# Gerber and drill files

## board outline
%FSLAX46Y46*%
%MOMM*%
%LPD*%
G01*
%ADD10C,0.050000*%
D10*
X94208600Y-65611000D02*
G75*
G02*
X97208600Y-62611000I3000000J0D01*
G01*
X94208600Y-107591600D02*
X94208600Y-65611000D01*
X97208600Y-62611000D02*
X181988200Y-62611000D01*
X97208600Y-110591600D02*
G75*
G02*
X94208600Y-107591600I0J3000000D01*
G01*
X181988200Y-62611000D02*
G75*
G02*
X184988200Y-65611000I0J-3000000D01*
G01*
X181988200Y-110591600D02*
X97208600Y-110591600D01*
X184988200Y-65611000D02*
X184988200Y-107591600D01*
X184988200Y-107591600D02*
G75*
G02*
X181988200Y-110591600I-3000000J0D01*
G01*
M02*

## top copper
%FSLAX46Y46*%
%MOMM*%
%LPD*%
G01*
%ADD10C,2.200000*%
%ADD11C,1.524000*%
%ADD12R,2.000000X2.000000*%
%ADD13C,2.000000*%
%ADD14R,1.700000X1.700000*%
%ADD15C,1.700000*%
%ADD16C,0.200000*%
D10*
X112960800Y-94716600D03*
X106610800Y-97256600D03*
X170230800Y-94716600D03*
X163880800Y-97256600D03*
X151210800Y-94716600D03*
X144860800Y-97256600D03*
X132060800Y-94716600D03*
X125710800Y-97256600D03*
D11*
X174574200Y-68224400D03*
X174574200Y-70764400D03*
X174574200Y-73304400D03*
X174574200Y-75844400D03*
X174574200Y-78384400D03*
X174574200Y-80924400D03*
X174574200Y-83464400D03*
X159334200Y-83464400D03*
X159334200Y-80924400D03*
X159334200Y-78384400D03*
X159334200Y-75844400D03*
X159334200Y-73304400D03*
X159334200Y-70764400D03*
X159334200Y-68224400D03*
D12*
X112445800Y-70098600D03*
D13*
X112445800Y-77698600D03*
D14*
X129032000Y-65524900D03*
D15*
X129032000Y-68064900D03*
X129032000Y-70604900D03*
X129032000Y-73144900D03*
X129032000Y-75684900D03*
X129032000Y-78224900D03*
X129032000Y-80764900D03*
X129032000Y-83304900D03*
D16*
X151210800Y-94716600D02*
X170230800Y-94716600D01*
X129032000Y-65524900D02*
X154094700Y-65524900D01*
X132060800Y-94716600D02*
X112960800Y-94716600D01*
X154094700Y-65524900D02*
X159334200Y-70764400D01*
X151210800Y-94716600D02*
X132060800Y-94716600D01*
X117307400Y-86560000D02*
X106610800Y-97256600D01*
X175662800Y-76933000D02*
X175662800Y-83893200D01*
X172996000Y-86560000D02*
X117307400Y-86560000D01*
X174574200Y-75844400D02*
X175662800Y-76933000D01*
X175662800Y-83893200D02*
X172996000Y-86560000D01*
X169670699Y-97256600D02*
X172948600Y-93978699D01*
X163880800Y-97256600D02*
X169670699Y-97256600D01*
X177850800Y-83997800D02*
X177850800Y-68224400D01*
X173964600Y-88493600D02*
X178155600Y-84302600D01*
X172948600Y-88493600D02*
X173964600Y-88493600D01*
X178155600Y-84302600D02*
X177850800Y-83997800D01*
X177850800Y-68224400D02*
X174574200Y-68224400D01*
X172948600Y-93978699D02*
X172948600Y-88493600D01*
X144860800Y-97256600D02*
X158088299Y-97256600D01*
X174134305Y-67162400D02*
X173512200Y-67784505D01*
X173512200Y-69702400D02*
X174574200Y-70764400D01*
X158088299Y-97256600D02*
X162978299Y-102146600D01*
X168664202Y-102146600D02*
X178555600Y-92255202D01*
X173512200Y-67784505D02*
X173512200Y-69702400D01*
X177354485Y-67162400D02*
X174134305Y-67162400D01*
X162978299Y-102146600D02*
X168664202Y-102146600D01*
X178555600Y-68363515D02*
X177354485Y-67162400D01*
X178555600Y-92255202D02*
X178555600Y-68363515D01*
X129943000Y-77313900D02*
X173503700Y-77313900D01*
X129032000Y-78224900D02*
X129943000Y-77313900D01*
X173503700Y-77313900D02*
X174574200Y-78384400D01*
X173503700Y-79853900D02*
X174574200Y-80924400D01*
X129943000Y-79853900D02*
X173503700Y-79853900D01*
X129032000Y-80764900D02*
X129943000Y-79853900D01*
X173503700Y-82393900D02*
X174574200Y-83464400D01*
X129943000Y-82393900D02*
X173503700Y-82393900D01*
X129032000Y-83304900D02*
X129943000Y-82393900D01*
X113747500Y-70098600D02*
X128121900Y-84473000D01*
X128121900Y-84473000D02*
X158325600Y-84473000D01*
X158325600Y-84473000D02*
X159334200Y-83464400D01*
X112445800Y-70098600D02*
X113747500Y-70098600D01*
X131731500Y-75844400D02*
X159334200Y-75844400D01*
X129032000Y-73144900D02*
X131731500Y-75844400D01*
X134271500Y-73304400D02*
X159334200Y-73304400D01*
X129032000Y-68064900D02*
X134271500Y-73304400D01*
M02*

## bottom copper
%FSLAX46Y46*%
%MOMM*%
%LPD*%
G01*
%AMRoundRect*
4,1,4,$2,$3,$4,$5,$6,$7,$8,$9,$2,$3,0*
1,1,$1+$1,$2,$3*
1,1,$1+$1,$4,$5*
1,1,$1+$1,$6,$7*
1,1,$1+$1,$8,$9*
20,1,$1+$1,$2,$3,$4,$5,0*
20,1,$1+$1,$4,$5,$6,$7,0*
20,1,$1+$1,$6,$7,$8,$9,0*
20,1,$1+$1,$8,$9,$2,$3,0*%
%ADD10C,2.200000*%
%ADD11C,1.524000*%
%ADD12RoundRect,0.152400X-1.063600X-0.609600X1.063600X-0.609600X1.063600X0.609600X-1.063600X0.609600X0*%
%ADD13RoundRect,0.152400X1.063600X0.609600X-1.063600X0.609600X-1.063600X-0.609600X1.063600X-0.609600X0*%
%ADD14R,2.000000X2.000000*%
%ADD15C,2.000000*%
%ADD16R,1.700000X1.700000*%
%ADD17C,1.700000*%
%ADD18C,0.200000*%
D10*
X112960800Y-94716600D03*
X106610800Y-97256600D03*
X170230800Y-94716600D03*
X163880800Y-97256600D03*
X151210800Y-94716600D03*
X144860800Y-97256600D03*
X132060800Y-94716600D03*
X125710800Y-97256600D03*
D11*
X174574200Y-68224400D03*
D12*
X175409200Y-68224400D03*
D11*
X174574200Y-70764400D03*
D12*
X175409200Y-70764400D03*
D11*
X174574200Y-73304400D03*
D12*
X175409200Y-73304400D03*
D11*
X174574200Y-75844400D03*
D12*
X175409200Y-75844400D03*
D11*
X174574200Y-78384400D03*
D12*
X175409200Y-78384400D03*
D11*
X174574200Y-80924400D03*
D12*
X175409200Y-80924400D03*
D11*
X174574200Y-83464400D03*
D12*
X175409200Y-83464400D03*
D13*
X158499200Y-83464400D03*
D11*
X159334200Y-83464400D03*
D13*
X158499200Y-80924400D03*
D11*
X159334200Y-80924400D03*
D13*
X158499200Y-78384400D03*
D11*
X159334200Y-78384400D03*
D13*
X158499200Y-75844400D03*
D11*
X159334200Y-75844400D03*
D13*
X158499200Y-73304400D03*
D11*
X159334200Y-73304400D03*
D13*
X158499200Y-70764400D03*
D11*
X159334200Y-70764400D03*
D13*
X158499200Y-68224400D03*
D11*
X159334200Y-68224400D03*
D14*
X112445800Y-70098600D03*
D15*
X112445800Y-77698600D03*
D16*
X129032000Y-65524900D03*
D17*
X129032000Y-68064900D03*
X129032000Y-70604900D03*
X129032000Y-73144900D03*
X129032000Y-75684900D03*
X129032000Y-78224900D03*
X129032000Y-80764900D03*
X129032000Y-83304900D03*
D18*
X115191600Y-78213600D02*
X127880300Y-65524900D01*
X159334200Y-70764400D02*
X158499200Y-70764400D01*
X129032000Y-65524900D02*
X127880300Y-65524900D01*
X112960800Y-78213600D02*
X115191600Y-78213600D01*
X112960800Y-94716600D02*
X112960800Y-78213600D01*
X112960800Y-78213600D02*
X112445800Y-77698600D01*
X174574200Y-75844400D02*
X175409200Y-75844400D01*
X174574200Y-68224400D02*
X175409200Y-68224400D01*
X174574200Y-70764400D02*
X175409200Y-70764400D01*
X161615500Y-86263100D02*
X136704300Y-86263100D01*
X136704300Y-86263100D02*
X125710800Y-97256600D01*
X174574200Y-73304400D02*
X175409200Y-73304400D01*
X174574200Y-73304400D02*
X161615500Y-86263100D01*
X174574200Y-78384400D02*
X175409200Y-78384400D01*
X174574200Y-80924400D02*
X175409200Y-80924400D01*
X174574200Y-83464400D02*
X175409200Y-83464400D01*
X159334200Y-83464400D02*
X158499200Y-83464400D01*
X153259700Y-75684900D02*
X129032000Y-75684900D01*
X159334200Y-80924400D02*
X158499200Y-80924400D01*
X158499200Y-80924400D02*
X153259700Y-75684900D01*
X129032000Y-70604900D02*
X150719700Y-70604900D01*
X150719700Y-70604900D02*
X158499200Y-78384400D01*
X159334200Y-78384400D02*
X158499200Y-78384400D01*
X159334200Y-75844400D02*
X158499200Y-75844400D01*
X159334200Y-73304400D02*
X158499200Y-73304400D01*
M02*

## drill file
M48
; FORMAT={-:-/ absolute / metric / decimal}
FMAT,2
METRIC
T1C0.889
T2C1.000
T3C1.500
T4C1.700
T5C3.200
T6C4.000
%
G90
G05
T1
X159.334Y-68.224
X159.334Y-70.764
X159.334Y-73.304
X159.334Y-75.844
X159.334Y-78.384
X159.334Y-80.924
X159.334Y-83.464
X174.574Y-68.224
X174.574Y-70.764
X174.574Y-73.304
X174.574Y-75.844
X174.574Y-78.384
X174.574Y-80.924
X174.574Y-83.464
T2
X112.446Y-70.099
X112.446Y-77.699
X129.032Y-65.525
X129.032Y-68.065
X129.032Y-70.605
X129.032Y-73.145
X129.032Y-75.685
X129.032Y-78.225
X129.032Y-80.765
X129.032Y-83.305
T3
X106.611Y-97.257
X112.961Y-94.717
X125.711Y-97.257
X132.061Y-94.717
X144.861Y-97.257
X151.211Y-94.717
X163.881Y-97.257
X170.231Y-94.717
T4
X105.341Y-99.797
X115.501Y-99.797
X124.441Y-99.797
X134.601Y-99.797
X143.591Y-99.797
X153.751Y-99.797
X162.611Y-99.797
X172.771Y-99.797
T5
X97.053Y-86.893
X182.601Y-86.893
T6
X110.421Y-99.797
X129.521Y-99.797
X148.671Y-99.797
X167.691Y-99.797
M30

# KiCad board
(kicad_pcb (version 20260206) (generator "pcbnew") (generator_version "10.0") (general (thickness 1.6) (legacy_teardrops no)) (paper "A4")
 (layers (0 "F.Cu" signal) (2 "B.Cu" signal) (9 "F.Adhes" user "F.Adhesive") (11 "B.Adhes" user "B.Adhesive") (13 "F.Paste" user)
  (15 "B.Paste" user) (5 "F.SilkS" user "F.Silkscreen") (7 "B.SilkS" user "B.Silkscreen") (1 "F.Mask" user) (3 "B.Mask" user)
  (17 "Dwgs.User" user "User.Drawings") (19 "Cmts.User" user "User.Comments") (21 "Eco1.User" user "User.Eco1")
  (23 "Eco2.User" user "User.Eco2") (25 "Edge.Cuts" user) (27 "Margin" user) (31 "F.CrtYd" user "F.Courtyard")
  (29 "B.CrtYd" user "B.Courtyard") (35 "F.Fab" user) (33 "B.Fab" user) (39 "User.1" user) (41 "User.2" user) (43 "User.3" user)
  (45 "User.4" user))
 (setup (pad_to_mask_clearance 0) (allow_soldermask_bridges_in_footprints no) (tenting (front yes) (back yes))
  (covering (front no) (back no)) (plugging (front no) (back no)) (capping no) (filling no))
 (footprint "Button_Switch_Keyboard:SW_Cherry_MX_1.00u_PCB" (layer "F.Cu") (at 112.9608 94.7166)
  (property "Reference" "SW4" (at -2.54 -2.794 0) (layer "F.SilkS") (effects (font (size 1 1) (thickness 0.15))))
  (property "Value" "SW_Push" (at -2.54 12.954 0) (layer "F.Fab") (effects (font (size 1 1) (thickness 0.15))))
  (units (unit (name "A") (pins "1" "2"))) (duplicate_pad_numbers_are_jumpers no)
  (pad "" np_thru_hole circle (at -7.62 5.08) (size 1.7 1.7) (drill 1.7) (layers "*.Cu" "*.Mask"))
  (pad "" np_thru_hole circle (at -2.54 5.08) (size 4 4) (drill 4) (layers "*.Cu" "*.Mask"))
  (pad "" np_thru_hole circle (at 2.54 5.08) (size 1.7 1.7) (drill 1.7) (layers "*.Cu" "*.Mask"))
  (pad "1" thru_hole circle (at 0 0) (size 2.2 2.2) (drill 1.5) (layers "*.Cu" "*.Mask") (remove_unused_layers no) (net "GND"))
  (pad "2" thru_hole circle (at -6.35 2.54) (size 2.2 2.2) (drill 1.5) (layers "*.Cu" "*.Mask") (remove_unused_layers no)
   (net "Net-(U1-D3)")))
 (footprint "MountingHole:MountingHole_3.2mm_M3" (layer "F.Cu") (at 97.0534 86.8934)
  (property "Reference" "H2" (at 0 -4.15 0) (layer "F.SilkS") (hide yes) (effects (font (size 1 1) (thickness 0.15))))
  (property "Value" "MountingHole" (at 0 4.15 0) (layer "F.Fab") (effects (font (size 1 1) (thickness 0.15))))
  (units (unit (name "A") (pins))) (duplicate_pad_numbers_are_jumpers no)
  (pad "" np_thru_hole circle (at 0 0) (size 3.2 3.2) (drill 3.2) (layers "*.Cu" "*.Mask")))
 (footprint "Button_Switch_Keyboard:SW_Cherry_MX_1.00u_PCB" (layer "F.Cu") (at 170.2308 94.7166)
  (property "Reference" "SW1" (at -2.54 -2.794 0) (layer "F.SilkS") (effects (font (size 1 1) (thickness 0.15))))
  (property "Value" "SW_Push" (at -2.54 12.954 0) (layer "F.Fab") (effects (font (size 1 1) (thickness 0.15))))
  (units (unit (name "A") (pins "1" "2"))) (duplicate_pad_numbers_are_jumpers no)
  (pad "" np_thru_hole circle (at -7.62 5.08) (size 1.7 1.7) (drill 1.7) (layers "*.Cu" "*.Mask"))
  (pad "" np_thru_hole circle (at -2.54 5.08) (size 4 4) (drill 4) (layers "*.Cu" "*.Mask"))
  (pad "" np_thru_hole circle (at 2.54 5.08) (size 1.7 1.7) (drill 1.7) (layers "*.Cu" "*.Mask"))
  (pad "1" thru_hole circle (at 0 0) (size 2.2 2.2) (drill 1.5) (layers "*.Cu" "*.Mask") (remove_unused_layers no) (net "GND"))
  (pad "2" thru_hole circle (at -6.35 2.54) (size 2.2 2.2) (drill 1.5) (layers "*.Cu" "*.Mask") (remove_unused_layers no)
   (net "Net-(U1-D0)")))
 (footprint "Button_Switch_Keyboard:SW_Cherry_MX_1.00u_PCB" (layer "F.Cu") (at 151.2108 94.7166)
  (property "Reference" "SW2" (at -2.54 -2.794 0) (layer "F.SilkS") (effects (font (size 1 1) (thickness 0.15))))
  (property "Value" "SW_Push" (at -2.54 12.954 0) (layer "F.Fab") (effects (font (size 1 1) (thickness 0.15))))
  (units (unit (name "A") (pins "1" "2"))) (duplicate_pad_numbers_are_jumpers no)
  (pad "" np_thru_hole circle (at -7.62 5.08) (size 1.7 1.7) (drill 1.7) (layers "*.Cu" "*.Mask"))
  (pad "" np_thru_hole circle (at -2.54 5.08) (size 4 4) (drill 4) (layers "*.Cu" "*.Mask"))
  (pad "" np_thru_hole circle (at 2.54 5.08) (size 1.7 1.7) (drill 1.7) (layers "*.Cu" "*.Mask"))
  (pad "1" thru_hole circle (at 0 0) (size 2.2 2.2) (drill 1.5) (layers "*.Cu" "*.Mask") (remove_unused_layers no) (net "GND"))
  (pad "2" thru_hole circle (at -6.35 2.54) (size 2.2 2.2) (drill 1.5) (layers "*.Cu" "*.Mask") (remove_unused_layers no)
   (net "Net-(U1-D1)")))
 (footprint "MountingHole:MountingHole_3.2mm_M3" (layer "F.Cu") (at 182.6006 86.8934)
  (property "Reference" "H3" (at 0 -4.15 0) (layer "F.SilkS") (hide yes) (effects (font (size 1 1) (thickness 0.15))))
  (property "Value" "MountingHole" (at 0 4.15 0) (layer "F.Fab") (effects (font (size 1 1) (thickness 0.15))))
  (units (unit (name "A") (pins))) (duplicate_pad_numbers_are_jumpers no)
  (pad "" np_thru_hole circle (at 0 0) (size 3.2 3.2) (drill 3.2) (layers "*.Cu" "*.Mask")))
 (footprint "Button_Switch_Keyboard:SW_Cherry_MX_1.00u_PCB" (layer "F.Cu") (at 132.0608 94.7166)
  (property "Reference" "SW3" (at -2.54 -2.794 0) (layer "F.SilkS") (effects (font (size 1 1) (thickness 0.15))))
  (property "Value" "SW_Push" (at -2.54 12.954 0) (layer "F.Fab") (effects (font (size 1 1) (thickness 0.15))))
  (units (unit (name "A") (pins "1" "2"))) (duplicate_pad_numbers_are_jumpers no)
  (pad "" np_thru_hole circle (at -7.62 5.08) (size 1.7 1.7) (drill 1.7) (layers "*.Cu" "*.Mask"))
  (pad "" np_thru_hole circle (at -2.54 5.08) (size 4 4) (drill 4) (layers "*.Cu" "*.Mask"))
  (pad "" np_thru_hole circle (at 2.54 5.08) (size 1.7 1.7) (drill 1.7) (layers "*.Cu" "*.Mask"))
  (pad "1" thru_hole circle (at 0 0) (size 2.2 2.2) (drill 1.5) (layers "*.Cu" "*.Mask") (remove_unused_layers no) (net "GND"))
  (pad "2" thru_hole circle (at -6.35 2.54) (size 2.2 2.2) (drill 1.5) (layers "*.Cu" "*.Mask") (remove_unused_layers no)
   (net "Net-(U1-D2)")))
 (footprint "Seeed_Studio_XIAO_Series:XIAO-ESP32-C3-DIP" (layer "B.Cu") (at 166.9542 75.8444 90)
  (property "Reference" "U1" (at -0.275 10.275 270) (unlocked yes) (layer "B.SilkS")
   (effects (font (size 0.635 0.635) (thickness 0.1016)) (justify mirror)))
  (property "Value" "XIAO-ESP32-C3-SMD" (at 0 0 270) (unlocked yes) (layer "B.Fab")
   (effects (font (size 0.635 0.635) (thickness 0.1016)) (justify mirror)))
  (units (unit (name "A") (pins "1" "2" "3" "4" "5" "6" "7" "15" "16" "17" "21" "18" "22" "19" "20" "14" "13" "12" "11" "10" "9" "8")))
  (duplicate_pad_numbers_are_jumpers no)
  (pad "1" thru_hole circle (at 7.62 7.62) (size 1.524 1.524) (drill 0.889) (layers "*.Cu" "*.Mask") (remove_unused_layers no)
   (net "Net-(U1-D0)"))
  (pad "1" smd roundrect (at 7.62 8.455) (size 2.432 1.524) (layers "B.Cu" "B.Mask") (roundrect_rratio 0.1) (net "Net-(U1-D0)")
   (thermal_bridge_angle 45))
  (pad "2" thru_hole circle (at 5.08 7.62) (size 1.524 1.524) (drill 0.889) (layers "*.Cu" "*.Mask") (remove_unused_layers no)
   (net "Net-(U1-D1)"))
  (pad "2" smd roundrect (at 5.08 8.455) (size 2.432 1.524) (layers "B.Cu" "B.Mask") (roundrect_rratio 0.1) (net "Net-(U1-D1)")
   (thermal_bridge_angle 45))
  (pad "3" thru_hole circle (at 2.54 7.62) (size 1.524 1.524) (drill 0.889) (layers "*.Cu" "*.Mask") (remove_unused_layers no)
   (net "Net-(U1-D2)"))
  (pad "3" smd roundrect (at 2.54 8.455) (size 2.432 1.524) (layers "B.Cu" "B.Mask") (roundrect_rratio 0.1) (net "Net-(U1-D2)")
   (thermal_bridge_angle 45))
  (pad "4" thru_hole circle (at 0 7.62) (size 1.524 1.524) (drill 0.889) (layers "*.Cu" "*.Mask") (remove_unused_layers no)
   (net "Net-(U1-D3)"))
  (pad "4" smd roundrect (at 0 8.455) (size 2.432 1.524) (layers "B.Cu" "B.Mask") (roundrect_rratio 0.1) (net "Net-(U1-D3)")
   (thermal_bridge_angle 45))
  (pad "5" thru_hole circle (at -2.54 7.62) (size 1.524 1.524) (drill 0.889) (layers "*.Cu" "*.Mask") (remove_unused_layers no) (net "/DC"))
  (pad "5" smd roundrect (at -2.54 8.455) (size 2.432 1.524) (layers "B.Cu" "B.Mask") (roundrect_rratio 0.1) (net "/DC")
   (thermal_bridge_angle 45))
  (pad "6" thru_hole circle (at -5.08 7.62) (size 1.524 1.524) (drill 0.889) (layers "*.Cu" "*.Mask") (remove_unused_layers no) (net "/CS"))
  (pad "6" smd roundrect (at -5.08 8.455) (size 2.432 1.524) (layers "B.Cu" "B.Mask") (roundrect_rratio 0.1) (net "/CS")
   (thermal_bridge_angle 45))
  (pad "7" thru_hole circle (at -7.62 7.62) (size 1.524 1.524) (drill 0.889) (layers "*.Cu" "*.Mask") (remove_unused_layers no) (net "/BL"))
  (pad "7" smd roundrect (at -7.62 8.455) (size 2.432 1.524) (layers "B.Cu" "B.Mask") (roundrect_rratio 0.1) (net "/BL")
   (thermal_bridge_angle 45))
  (pad "8" smd roundrect (at -7.62 -8.455 180) (size 2.432 1.524) (layers "B.Cu" "B.Mask") (roundrect_rratio 0.1) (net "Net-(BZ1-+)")
   (thermal_bridge_angle 45))
  (pad "8" thru_hole circle (at -7.62 -7.62 180) (size 1.524 1.524) (drill 0.889) (layers "*.Cu" "*.Mask") (remove_unused_layers no)
   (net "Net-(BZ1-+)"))
  (pad "9" smd roundrect (at -5.08 -8.455 180) (size 2.432 1.524) (layers "B.Cu" "B.Mask") (roundrect_rratio 0.1) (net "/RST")
   (thermal_bridge_angle 45))
  (pad "9" thru_hole circle (at -5.08 -7.62 180) (size 1.524 1.524) (drill 0.889) (layers "*.Cu" "*.Mask") (remove_unused_layers no)
   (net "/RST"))
  (pad "10" smd roundrect (at -2.54 -8.455 180) (size 2.432 1.524) (layers "B.Cu" "B.Mask") (roundrect_rratio 0.1) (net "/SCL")
   (thermal_bridge_angle 45))
  (pad "10" thru_hole circle (at -2.54 -7.62 180) (size 1.524 1.524) (drill 0.889) (layers "*.Cu" "*.Mask") (remove_unused_layers no)
   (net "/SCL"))
  (pad "11" smd roundrect (at 0 -8.455 180) (size 2.432 1.524) (layers "B.Cu" "B.Mask") (roundrect_rratio 0.1) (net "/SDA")
   (thermal_bridge_angle 45))
  (pad "11" thru_hole circle (at 0 -7.62 180) (size 1.524 1.524) (drill 0.889) (layers "*.Cu" "*.Mask") (remove_unused_layers no)
   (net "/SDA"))
  (pad "12" smd roundrect (at 2.54 -8.455 180) (size 2.432 1.524) (layers "B.Cu" "B.Mask") (roundrect_rratio 0.1) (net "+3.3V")
   (thermal_bridge_angle 45))
  (pad "12" thru_hole circle (at 2.54 -7.62 180) (size 1.524 1.524) (drill 0.889) (layers "*.Cu" "*.Mask") (remove_unused_layers no)
   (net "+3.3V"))
  (pad "13" smd roundrect (at 5.08 -8.455 180) (size 2.432 1.524) (layers "B.Cu" "B.Mask") (roundrect_rratio 0.1) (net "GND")
   (thermal_bridge_angle 45))
  (pad "13" thru_hole circle (at 5.08 -7.62 180) (size 1.524 1.524) (drill 0.889) (layers "*.Cu" "*.Mask") (remove_unused_layers no)
   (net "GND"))
  (pad "14" smd roundrect (at 7.62 -8.455 180) (size 2.432 1.524) (layers "B.Cu" "B.Mask") (roundrect_rratio 0.1)
   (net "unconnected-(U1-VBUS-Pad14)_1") (thermal_bridge_angle 45))
  (pad "14" thru_hole circle (at 7.62 -7.62 180) (size 1.524 1.524) (drill 0.889) (layers "*.Cu" "*.Mask") (remove_unused_layers no)
   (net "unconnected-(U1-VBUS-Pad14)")))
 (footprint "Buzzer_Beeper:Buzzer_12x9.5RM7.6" (layer "B.Cu") (at 112.4458 70.0986 -90)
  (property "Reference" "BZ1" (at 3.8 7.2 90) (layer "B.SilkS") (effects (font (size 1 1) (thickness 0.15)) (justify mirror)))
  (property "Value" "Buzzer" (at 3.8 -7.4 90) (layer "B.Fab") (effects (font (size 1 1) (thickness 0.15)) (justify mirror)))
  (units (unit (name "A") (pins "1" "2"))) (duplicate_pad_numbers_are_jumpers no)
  (pad "1" thru_hole rect (at 0 0 270) (size 2 2) (drill 1) (layers "*.Cu" "*.Mask") (remove_unused_layers no) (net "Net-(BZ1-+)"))
  (pad "2" thru_hole circle (at 7.6 0 270) (size 2 2) (drill 1) (layers "*.Cu" "*.Mask") (remove_unused_layers no) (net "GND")))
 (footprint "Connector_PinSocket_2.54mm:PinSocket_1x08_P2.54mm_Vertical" (layer "B.Cu") (at 129.032 65.5249 180)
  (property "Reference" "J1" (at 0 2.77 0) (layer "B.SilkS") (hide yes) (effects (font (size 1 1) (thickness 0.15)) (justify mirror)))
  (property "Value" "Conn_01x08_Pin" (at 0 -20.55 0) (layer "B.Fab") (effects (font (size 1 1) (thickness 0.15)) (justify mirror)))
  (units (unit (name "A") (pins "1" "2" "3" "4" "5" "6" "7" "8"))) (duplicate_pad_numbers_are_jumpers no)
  (pad "1" thru_hole rect (at 0 0 180) (size 1.7 1.7) (drill 1) (layers "*.Cu" "*.Mask") (remove_unused_layers no) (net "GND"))
  (pad "2" thru_hole circle (at 0 -2.54 180) (size 1.7 1.7) (drill 1) (layers "*.Cu" "*.Mask") (remove_unused_layers no) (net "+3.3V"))
  (pad "3" thru_hole circle (at 0 -5.08 180) (size 1.7 1.7) (drill 1) (layers "*.Cu" "*.Mask") (remove_unused_layers no) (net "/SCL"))
  (pad "4" thru_hole circle (at 0 -7.62 180) (size 1.7 1.7) (drill 1) (layers "*.Cu" "*.Mask") (remove_unused_layers no) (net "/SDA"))
  (pad "5" thru_hole circle (at 0 -10.16 180) (size 1.7 1.7) (drill 1) (layers "*.Cu" "*.Mask") (remove_unused_layers no) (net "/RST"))
  (pad "6" thru_hole circle (at 0 -12.7 180) (size 1.7 1.7) (drill 1) (layers "*.Cu" "*.Mask") (remove_unused_layers no) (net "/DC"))
  (pad "7" thru_hole circle (at 0 -15.24 180) (size 1.7 1.7) (drill 1) (layers "*.Cu" "*.Mask") (remove_unused_layers no) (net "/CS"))
  (pad "8" thru_hole circle (at 0 -17.78 180) (size 1.7 1.7) (drill 1) (layers "*.Cu" "*.Mask") (remove_unused_layers no) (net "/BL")))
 (gr_arc (start 94.2086 65.611) (mid 95.08728 63.48968) (end 97.2086 62.611) (stroke (width 0.05) (type default)) (layer "Edge.Cuts"))
 (gr_line (start 94.2086 107.5916) (end 94.2086 65.611) (stroke (width 0.05) (type default)) (layer "Edge.Cuts"))
 (gr_line (start 97.2086 62.611) (end 181.9882 62.611) (stroke (width 0.05) (type default)) (layer "Edge.Cuts"))
 (gr_arc (start 97.2086 110.5916) (mid 95.08728 109.71292) (end 94.2086 107.5916) (stroke (width 0.05) (type default)) (layer "Edge.Cuts"))
 (gr_arc (start 181.9882 62.611) (mid 184.10952 63.48968) (end 184.9882 65.611) (stroke (width 0.05) (type default)) (layer "Edge.Cuts"))
 (gr_line (start 181.9882 110.5916) (end 97.2086 110.5916) (stroke (width 0.05) (type default)) (layer "Edge.Cuts"))
 (gr_line (start 184.9882 65.611) (end 184.9882 107.5916) (stroke (width 0.05) (type default)) (layer "Edge.Cuts"))
 (gr_arc (start 184.9882 107.5916) (mid 184.10952 109.71292) (end 181.9882 110.5916) (stroke (width 0.05) (type default))
  (layer "Edge.Cuts"))
 (segment (start 151.2108 94.7166) (end 170.2308 94.7166) (width 0.2) (layer "F.Cu") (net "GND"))
 (segment (start 129.032 65.5249) (end 154.0947 65.5249) (width 0.2) (layer "F.Cu") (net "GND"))
 (segment (start 132.0608 94.7166) (end 112.9608 94.7166) (width 0.2) (layer "F.Cu") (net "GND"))
 (segment (start 154.0947 65.5249) (end 159.3342 70.7644) (width 0.2) (layer "F.Cu") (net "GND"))
 (segment (start 151.2108 94.7166) (end 132.0608 94.7166) (width 0.2) (layer "F.Cu") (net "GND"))
 (segment (start 115.1916 78.2136) (end 127.8803 65.5249) (width 0.2) (layer "B.Cu") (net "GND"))
 (segment (start 159.3342 70.7644) (end 158.4992 70.7644) (width 0.2) (layer "B.Cu") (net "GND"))
 (segment (start 129.032 65.5249) (end 127.8803 65.5249) (width 0.2) (layer "B.Cu") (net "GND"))
 (segment (start 112.9608 78.2136) (end 115.1916 78.2136) (width 0.2) (layer "B.Cu") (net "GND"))
 (segment (start 112.9608 94.7166) (end 112.9608 78.2136) (width 0.2) (layer "B.Cu") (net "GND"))
 (segment (start 112.9608 78.2136) (end 112.4458 77.6986) (width 0.2) (layer "B.Cu") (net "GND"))
 (segment (start 117.3074 86.56) (end 106.6108 97.2566) (width 0.2) (layer "F.Cu") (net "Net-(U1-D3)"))
 (segment (start 175.6628 76.933) (end 175.6628 83.8932) (width 0.2) (layer "F.Cu") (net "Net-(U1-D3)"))
 (segment (start 172.996 86.56) (end 117.3074 86.56) (width 0.2) (layer "F.Cu") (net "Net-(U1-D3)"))
 (segment (start 174.5742 75.8444) (end 175.6628 76.933) (width 0.2) (layer "F.Cu") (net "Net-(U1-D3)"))
 (segment (start 175.6628 83.8932) (end 172.996 86.56) (width 0.2) (layer "F.Cu") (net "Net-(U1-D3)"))
 (segment (start 174.5742 75.8444) (end 175.4092 75.8444) (width 0.2) (layer "B.Cu") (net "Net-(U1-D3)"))
 (segment (start 169.670699 97.2566) (end 172.9486 93.978699) (width 0.2) (layer "F.Cu") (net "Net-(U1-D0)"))
 (segment (start 163.8808 97.2566) (end 169.670699 97.2566) (width 0.2) (layer "F.Cu") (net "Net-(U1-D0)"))
 (segment (start 177.8508 83.9978) (end 177.8508 68.2244) (width 0.2) (layer "F.Cu") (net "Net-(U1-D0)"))
 (segment (start 173.9646 88.4936) (end 178.1556 84.3026) (width 0.2) (layer "F.Cu") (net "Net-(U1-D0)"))
 (segment (start 172.9486 88.4936) (end 173.9646 88.4936) (width 0.2) (layer "F.Cu") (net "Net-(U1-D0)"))
 (segment (start 178.1556 84.3026) (end 177.8508 83.9978) (width 0.2) (layer "F.Cu") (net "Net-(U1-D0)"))
 (segment (start 177.8508 68.2244) (end 174.5742 68.2244) (width 0.2) (layer "F.Cu") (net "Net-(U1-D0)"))
 (segment (start 172.9486 93.978699) (end 172.9486 88.4936) (width 0.2) (layer "F.Cu") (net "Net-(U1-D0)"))
 (segment (start 174.5742 68.2244) (end 175.4092 68.2244) (width 0.2) (layer "B.Cu") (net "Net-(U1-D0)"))
 (segment (start 144.8608 97.2566) (end 158.088299 97.2566) (width 0.2) (layer "F.Cu") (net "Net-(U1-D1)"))
 (segment (start 174.134305 67.1624) (end 173.5122 67.784505) (width 0.2) (layer "F.Cu") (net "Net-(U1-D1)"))
 (segment (start 173.5122 69.7024) (end 174.5742 70.7644) (width 0.2) (layer "F.Cu") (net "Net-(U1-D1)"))
 (segment (start 158.088299 97.2566) (end 162.978299 102.1466) (width 0.2) (layer "F.Cu") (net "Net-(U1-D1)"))
 (segment (start 168.664202 102.1466) (end 178.5556 92.255202) (width 0.2) (layer "F.Cu") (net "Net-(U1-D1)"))
 (segment (start 173.5122 67.784505) (end 173.5122 69.7024) (width 0.2) (layer "F.Cu") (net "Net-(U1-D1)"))
 (segment (start 177.354485 67.1624) (end 174.134305 67.1624) (width 0.2) (layer "F.Cu") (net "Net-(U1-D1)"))
 (segment (start 162.978299 102.1466) (end 168.664202 102.1466) (width 0.2) (layer "F.Cu") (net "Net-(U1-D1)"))
 (segment (start 178.5556 68.363515) (end 177.354485 67.1624) (width 0.2) (layer "F.Cu") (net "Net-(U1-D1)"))
 (segment (start 178.5556 92.255202) (end 178.5556 68.363515) (width 0.2) (layer "F.Cu") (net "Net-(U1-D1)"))
 (segment (start 174.5742 70.7644) (end 175.4092 70.7644) (width 0.2) (layer "B.Cu") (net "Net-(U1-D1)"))
 (segment (start 161.6155 86.2631) (end 136.7043 86.2631) (width 0.2) (layer "B.Cu") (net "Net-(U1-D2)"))
 (segment (start 136.7043 86.2631) (end 125.7108 97.2566) (width 0.2) (layer "B.Cu") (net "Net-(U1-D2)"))
 (segment (start 174.5742 73.3044) (end 175.4092 73.3044) (width 0.2) (layer "B.Cu") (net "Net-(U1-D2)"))
 (segment (start 174.5742 73.3044) (end 161.6155 86.2631) (width 0.2) (layer "B.Cu") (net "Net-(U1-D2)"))
 (segment (start 129.943 77.3139) (end 173.5037 77.3139) (width 0.2) (layer "F.Cu") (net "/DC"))
 (segment (start 129.032 78.2249) (end 129.943 77.3139) (width 0.2) (layer "F.Cu") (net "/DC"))
 (segment (start 173.5037 77.3139) (end 174.5742 78.3844) (width 0.2) (layer "F.Cu") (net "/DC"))
 (segment (start 174.5742 78.3844) (end 175.4092 78.3844) (width 0.2) (layer "B.Cu") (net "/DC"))
 (segment (start 173.5037 79.8539) (end 174.5742 80.9244) (width 0.2) (layer "F.Cu") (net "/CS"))
 (segment (start 129.943 79.8539) (end 173.5037 79.8539) (width 0.2) (layer "F.Cu") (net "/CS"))
 (segment (start 129.032 80.7649) (end 129.943 79.8539) (width 0.2) (layer "F.Cu") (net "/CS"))
 (segment (start 174.5742 80.9244) (end 175.4092 80.9244) (width 0.2) (layer "B.Cu") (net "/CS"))
 (segment (start 173.5037 82.3939) (end 174.5742 83.4644) (width 0.2) (layer "F.Cu") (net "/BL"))
 (segment (start 129.943 82.3939) (end 173.5037 82.3939) (width 0.2) (layer "F.Cu") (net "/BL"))
 (segment (start 129.032 83.3049) (end 129.943 82.3939) (width 0.2) (layer "F.Cu") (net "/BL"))
 (segment (start 174.5742 83.4644) (end 175.4092 83.4644) (width 0.2) (layer "B.Cu") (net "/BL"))
 (segment (start 113.7475 70.0986) (end 128.1219 84.473) (width 0.2) (layer "F.Cu") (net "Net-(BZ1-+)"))
 (segment (start 128.1219 84.473) (end 158.3256 84.473) (width 0.2) (layer "F.Cu") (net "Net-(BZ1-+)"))
 (segment (start 158.3256 84.473) (end 159.3342 83.4644) (width 0.2) (layer "F.Cu") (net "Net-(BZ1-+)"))
 (segment (start 112.4458 70.0986) (end 113.7475 70.0986) (width 0.2) (layer "F.Cu") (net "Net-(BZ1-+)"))
 (segment (start 159.3342 83.4644) (end 158.4992 83.4644) (width 0.2) (layer "B.Cu") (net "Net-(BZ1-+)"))
 (segment (start 153.2597 75.6849) (end 129.032 75.6849) (width 0.2) (layer "B.Cu") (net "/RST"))
 (segment (start 159.3342 80.9244) (end 158.4992 80.9244) (width 0.2) (layer "B.Cu") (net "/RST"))
 (segment (start 158.4992 80.9244) (end 153.2597 75.6849) (width 0.2) (layer "B.Cu") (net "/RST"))
 (segment (start 129.032 70.6049) (end 150.7197 70.6049) (width 0.2) (layer "B.Cu") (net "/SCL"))
 (segment (start 150.7197 70.6049) (end 158.4992 78.3844) (width 0.2) (layer "B.Cu") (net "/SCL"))
 (segment (start 159.3342 78.3844) (end 158.4992 78.3844) (width 0.2) (layer "B.Cu") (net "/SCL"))
 (segment (start 131.7315 75.8444) (end 159.3342 75.8444) (width 0.2) (layer "F.Cu") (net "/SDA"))
 (segment (start 129.032 73.1449) (end 131.7315 75.8444) (width 0.2) (layer "F.Cu") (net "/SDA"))
 (segment (start 159.3342 75.8444) (end 158.4992 75.8444) (width 0.2) (layer "B.Cu") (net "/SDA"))
 (segment (start 134.2715 73.3044) (end 159.3342 73.3044) (width 0.2) (layer "F.Cu") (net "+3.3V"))
 (segment (start 129.032 68.0649) (end 134.2715 73.3044) (width 0.2) (layer "F.Cu") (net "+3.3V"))
 (segment (start 159.3342 73.3044) (end 158.4992 73.3044) (width 0.2) (layer "B.Cu") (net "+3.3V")))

